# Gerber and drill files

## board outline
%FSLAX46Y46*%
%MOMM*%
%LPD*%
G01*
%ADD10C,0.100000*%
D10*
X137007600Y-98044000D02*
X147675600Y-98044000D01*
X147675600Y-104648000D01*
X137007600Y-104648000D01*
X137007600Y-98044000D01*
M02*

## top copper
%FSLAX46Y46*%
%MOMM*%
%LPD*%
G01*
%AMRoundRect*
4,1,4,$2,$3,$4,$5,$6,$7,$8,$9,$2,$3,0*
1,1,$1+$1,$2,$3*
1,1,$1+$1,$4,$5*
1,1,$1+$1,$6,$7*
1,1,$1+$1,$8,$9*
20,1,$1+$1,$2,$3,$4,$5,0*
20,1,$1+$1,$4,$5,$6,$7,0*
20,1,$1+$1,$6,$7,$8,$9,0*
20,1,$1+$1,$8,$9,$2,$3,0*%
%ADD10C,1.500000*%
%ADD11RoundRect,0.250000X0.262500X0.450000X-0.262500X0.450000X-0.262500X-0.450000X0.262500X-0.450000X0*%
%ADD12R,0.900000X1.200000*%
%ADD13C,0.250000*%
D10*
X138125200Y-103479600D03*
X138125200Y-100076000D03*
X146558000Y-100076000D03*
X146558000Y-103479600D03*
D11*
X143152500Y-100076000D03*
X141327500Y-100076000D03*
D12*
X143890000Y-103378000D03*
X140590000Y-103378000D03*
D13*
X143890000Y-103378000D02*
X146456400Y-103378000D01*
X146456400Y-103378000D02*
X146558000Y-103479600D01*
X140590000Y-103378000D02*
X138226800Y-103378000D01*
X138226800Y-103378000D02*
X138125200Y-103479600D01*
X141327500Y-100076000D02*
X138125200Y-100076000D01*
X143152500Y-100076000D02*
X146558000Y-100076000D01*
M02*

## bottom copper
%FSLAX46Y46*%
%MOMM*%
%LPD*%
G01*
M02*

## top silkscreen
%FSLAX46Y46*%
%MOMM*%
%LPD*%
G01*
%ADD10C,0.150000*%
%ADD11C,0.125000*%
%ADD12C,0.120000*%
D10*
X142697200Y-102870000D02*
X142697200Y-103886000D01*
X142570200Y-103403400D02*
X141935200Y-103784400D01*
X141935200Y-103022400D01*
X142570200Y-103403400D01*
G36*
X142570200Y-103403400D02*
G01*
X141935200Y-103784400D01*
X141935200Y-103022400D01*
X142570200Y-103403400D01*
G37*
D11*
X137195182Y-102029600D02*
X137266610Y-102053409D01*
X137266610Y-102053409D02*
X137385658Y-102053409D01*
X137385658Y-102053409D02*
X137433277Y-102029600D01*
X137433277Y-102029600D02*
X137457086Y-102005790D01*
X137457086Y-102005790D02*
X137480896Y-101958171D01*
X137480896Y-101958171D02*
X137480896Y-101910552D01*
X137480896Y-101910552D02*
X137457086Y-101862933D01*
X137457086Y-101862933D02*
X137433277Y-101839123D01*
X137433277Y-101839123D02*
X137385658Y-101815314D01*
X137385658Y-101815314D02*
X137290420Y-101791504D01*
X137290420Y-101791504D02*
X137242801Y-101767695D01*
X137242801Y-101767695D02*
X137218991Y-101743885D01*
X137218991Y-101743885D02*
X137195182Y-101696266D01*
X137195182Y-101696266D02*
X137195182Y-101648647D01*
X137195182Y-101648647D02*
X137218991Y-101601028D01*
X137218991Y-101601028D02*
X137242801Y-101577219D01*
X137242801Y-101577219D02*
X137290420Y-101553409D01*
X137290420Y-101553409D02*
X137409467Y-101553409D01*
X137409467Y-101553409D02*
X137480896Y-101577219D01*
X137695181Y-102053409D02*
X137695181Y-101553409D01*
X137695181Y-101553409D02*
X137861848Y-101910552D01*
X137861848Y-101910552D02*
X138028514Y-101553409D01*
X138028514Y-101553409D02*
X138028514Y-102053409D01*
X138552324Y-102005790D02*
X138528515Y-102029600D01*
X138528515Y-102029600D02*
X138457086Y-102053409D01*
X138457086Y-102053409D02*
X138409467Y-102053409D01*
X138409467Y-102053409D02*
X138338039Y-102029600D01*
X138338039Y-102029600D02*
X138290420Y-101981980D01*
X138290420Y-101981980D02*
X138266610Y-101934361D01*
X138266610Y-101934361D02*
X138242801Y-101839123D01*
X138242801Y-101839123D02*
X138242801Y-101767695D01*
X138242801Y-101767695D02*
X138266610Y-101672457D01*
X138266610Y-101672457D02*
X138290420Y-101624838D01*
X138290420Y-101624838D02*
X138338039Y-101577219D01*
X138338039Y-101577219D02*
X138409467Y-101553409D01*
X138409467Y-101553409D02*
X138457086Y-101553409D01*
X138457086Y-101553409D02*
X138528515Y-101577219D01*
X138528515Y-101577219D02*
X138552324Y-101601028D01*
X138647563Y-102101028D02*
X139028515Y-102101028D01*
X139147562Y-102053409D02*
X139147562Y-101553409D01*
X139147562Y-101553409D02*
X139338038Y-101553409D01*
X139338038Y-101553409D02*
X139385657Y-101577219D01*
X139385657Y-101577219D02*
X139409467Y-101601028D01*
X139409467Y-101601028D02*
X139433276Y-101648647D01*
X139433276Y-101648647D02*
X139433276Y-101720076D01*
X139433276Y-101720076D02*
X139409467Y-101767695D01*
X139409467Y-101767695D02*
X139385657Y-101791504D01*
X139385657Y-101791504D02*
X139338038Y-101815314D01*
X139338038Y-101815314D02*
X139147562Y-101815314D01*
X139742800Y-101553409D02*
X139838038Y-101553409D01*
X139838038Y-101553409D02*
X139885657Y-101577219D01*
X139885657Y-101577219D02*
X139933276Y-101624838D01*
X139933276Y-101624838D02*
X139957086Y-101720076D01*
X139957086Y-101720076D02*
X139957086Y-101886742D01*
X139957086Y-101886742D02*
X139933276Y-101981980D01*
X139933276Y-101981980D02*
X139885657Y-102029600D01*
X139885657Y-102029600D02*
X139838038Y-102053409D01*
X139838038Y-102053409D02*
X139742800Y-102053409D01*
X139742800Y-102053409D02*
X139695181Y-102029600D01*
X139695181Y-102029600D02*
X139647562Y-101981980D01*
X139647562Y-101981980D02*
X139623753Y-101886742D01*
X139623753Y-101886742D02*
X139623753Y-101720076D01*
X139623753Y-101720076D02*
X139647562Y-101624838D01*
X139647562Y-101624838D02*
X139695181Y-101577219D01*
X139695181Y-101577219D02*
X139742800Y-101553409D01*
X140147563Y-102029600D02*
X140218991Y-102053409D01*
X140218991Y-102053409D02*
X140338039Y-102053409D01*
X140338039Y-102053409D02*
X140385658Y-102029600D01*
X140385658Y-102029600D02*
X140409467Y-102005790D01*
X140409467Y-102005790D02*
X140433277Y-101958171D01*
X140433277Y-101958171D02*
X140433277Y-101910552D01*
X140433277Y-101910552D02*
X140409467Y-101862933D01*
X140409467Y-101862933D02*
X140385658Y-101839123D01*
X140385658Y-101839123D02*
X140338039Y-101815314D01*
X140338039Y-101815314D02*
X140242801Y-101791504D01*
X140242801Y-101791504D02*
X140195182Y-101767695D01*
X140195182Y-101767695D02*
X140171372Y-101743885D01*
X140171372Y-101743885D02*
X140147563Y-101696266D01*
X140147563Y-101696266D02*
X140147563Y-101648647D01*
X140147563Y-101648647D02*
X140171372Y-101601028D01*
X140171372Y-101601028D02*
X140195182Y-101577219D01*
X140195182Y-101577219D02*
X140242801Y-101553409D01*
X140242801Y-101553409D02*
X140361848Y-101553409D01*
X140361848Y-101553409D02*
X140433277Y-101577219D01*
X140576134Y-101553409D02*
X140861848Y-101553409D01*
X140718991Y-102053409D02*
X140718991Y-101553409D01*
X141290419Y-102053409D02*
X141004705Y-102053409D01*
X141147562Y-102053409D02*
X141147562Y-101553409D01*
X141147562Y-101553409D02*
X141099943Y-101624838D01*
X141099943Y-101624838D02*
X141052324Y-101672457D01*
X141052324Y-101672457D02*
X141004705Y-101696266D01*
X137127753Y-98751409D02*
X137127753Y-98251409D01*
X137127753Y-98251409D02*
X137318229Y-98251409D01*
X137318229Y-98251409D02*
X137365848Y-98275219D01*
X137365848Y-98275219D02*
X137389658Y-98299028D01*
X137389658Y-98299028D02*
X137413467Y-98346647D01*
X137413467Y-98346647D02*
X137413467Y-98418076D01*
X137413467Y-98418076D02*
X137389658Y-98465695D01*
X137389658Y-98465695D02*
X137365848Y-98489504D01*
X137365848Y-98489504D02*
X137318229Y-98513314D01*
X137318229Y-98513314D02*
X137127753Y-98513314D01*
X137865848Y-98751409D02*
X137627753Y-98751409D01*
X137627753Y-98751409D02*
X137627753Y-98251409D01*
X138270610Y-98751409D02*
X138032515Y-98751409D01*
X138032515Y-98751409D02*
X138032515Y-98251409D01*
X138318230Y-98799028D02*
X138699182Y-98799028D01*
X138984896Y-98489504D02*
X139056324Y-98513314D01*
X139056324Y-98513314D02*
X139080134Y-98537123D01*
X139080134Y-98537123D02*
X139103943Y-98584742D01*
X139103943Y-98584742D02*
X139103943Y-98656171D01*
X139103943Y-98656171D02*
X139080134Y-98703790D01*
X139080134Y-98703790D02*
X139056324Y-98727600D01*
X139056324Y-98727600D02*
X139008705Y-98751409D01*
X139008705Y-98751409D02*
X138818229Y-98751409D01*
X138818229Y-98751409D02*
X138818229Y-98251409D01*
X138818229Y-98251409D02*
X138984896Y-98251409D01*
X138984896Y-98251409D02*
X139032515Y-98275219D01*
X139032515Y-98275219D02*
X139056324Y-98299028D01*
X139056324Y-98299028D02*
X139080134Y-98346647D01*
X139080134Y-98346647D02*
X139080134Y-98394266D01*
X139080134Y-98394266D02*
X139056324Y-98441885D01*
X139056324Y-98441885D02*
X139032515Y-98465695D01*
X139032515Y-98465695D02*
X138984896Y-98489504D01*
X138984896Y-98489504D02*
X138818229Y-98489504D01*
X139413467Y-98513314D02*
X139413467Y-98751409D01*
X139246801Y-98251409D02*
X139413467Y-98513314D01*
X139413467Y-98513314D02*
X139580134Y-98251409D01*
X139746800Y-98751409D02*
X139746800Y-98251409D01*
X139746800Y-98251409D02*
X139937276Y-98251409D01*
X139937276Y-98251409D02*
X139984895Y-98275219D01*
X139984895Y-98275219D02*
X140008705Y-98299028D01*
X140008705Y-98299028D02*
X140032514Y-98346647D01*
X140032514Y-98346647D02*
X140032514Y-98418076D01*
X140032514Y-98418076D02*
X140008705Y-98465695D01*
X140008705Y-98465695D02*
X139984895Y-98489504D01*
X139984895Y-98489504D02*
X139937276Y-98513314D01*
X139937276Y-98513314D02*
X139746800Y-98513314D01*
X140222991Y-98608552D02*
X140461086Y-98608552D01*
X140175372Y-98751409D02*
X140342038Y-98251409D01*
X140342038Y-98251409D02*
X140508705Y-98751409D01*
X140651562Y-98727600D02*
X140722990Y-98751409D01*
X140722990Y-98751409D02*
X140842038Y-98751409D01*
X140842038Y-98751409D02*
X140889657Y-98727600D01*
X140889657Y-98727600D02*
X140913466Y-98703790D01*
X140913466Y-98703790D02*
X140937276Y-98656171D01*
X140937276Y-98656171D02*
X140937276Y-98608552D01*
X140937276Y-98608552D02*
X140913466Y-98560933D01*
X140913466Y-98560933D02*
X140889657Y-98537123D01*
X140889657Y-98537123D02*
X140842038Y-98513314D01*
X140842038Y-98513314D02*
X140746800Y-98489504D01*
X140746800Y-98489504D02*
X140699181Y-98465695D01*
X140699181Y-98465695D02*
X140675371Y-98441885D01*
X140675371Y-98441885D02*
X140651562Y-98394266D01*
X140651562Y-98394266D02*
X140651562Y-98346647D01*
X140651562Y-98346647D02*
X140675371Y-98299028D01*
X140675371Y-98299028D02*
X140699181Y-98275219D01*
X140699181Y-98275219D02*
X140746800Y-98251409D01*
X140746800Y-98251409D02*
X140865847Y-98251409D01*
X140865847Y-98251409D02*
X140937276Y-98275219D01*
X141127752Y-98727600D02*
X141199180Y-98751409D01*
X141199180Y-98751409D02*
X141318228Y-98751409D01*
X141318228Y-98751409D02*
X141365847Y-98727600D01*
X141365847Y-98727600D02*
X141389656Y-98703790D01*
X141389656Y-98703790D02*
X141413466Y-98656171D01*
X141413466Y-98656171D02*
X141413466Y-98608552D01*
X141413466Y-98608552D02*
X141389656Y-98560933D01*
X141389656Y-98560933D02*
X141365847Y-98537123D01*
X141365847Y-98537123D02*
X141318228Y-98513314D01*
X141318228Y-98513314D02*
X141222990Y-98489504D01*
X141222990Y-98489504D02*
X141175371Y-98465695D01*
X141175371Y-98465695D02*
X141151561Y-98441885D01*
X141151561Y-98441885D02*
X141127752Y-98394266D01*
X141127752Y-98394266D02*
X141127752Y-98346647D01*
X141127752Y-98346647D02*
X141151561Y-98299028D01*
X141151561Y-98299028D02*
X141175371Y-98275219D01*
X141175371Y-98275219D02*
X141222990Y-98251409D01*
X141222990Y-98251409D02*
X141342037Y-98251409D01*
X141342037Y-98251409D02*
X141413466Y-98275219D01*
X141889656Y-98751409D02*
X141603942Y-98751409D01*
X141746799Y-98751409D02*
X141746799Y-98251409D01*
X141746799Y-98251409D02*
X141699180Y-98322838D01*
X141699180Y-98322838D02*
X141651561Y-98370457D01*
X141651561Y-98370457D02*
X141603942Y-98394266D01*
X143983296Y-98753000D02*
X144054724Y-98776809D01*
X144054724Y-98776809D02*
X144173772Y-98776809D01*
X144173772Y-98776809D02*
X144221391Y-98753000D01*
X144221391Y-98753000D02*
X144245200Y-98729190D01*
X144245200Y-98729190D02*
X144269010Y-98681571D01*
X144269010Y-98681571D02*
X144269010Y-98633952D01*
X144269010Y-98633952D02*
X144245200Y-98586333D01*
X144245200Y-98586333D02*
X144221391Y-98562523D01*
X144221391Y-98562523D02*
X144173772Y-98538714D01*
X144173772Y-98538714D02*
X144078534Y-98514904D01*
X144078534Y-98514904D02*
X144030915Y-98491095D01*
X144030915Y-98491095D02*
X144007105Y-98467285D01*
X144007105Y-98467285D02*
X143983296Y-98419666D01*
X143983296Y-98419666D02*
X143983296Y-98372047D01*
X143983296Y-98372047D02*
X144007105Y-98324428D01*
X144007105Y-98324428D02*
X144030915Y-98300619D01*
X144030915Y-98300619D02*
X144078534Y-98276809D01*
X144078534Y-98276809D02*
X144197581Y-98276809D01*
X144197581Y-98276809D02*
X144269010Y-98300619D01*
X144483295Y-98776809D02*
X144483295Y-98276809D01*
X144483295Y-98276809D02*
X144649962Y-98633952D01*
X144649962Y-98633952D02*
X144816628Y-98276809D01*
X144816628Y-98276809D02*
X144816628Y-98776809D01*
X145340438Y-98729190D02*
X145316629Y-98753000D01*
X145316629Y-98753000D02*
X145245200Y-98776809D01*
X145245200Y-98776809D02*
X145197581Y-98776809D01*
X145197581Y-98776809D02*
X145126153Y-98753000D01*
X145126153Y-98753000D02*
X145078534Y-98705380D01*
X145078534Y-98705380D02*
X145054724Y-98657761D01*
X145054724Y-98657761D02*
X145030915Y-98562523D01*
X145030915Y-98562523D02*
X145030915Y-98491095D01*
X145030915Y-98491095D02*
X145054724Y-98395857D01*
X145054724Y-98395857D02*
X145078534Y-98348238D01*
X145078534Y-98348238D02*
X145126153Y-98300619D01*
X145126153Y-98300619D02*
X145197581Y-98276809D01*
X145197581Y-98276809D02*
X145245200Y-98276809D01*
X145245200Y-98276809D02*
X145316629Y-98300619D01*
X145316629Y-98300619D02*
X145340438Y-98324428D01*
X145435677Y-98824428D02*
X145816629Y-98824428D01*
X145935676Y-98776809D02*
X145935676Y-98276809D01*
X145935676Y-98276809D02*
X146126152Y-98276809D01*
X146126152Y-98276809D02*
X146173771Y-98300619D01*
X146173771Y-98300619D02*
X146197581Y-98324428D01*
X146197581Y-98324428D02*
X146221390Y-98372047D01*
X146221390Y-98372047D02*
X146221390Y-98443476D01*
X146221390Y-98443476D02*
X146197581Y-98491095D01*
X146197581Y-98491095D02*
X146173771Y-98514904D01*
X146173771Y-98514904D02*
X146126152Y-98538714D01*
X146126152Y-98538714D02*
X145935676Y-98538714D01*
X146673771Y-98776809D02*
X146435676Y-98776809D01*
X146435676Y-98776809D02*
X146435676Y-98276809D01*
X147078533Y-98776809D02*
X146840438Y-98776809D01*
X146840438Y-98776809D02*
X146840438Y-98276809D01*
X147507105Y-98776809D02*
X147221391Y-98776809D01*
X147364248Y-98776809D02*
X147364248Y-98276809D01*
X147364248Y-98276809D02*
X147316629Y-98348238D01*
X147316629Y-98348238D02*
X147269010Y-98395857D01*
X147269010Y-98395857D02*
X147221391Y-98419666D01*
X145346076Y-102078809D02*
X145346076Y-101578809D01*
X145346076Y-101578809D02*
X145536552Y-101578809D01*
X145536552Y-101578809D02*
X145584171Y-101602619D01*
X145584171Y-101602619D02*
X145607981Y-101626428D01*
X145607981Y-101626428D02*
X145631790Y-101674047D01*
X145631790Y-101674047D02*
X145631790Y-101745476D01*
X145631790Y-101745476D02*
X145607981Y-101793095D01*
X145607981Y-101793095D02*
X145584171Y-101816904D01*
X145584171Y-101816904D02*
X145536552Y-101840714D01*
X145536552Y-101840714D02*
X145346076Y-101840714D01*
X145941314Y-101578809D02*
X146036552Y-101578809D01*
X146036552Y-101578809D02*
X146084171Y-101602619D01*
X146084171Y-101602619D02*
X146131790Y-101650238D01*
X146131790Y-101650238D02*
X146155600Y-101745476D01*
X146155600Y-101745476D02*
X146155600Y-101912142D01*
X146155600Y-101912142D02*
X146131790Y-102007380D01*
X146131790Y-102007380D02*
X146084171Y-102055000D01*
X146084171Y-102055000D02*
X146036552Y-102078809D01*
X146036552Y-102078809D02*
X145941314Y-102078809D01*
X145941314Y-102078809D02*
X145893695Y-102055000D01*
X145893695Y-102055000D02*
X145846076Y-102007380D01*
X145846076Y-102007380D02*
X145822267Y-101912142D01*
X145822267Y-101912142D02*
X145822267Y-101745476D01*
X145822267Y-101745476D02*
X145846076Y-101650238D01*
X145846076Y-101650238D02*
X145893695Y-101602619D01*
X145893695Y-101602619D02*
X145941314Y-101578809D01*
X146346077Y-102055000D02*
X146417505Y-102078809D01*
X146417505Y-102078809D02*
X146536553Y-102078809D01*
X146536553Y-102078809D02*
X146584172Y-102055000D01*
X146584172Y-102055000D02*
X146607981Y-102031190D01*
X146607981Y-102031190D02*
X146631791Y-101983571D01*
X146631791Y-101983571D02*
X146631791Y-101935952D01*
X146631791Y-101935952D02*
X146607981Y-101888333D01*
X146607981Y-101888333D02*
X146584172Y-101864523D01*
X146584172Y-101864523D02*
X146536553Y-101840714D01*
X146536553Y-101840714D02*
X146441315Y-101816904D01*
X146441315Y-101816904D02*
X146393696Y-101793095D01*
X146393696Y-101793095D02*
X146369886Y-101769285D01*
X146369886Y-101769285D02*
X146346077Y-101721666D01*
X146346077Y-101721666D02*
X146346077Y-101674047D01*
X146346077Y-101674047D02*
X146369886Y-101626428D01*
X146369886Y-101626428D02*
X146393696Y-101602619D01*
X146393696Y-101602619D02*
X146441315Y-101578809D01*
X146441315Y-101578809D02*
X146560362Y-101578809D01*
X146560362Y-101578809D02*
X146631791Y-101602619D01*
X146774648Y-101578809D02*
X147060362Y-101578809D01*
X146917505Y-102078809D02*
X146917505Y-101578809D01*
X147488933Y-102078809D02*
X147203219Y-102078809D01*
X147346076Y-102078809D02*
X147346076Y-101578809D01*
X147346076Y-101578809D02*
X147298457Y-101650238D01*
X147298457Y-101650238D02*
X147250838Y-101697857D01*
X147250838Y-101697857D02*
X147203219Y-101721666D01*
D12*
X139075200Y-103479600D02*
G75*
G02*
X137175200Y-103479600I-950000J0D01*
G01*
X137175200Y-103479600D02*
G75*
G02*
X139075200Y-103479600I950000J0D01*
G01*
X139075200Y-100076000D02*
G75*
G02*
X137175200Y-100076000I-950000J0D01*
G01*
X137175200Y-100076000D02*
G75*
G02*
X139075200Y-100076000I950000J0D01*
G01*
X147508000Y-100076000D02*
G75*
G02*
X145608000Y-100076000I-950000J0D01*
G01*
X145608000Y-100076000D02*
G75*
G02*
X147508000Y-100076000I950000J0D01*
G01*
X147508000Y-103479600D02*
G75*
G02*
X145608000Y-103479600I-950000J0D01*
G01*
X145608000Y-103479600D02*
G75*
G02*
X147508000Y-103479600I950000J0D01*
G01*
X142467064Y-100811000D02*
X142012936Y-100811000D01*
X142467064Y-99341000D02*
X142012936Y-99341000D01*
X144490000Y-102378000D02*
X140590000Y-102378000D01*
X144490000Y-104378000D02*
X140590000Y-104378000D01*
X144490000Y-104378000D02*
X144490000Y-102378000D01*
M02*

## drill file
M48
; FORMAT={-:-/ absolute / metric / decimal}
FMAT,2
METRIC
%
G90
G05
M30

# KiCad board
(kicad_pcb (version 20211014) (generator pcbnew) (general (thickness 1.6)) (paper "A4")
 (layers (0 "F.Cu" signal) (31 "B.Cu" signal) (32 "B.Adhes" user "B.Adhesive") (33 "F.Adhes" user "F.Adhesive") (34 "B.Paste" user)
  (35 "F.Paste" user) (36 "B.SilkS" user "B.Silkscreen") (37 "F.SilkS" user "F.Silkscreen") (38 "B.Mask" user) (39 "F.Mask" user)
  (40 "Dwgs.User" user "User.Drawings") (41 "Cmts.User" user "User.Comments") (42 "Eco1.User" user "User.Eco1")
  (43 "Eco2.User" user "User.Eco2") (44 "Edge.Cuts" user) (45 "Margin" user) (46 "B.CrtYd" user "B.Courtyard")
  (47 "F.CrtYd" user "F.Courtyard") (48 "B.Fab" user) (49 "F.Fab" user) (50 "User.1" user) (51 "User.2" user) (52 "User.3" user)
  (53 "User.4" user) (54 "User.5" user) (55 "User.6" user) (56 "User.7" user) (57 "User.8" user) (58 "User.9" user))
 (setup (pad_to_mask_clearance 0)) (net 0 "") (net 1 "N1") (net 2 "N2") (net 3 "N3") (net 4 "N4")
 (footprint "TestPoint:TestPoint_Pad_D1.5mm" (layer "F.Cu") (at 138.1252 103.4796)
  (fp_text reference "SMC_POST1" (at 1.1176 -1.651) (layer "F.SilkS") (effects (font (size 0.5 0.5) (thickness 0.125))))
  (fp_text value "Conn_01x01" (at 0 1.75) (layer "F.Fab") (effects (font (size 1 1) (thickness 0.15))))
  (fp_circle (center 0 0) (end 0 0.95) (layer "F.SilkS") (width 0.12) (fill none))
  (pad "1" smd circle (at 0 0) (size 1.5 1.5) (layers "F.Cu" "F.Mask") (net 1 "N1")))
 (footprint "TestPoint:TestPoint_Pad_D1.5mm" (layer "F.Cu") (at 138.1252 100.076)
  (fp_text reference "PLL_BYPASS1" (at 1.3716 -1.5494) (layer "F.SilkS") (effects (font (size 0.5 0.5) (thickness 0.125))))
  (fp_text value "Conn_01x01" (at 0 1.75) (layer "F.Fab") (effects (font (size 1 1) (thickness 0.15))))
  (fp_circle (center 0 0) (end 0 0.95) (layer "F.SilkS") (width 0.12) (fill none))
  (pad "1" smd circle (at 0 0) (size 1.5 1.5) (layers "F.Cu" "F.Mask") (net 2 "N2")))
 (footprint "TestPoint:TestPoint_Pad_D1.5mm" (layer "F.Cu") (at 146.558 100.076)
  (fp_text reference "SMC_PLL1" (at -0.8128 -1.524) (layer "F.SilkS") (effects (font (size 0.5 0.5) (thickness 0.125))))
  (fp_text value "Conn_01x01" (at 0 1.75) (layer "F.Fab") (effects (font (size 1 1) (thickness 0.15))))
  (fp_circle (center 0 0) (end 0 0.95) (layer "F.SilkS") (width 0.12) (fill none))
  (pad "1" smd circle (at 0 0) (size 1.5 1.5) (layers "F.Cu" "F.Mask") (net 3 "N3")))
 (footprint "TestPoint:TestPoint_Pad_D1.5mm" (layer "F.Cu") (at 146.558 103.4796)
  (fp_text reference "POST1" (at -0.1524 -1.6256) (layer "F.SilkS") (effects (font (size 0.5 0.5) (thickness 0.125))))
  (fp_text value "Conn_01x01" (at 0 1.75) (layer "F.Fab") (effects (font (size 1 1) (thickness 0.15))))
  (fp_circle (center 0 0) (end 0 0.95) (layer "F.SilkS") (width 0.12) (fill none))
  (pad "1" smd circle (at 0 0) (size 1.5 1.5) (layers "F.Cu" "F.Mask") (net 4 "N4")))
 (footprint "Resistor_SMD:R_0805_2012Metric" (layer "F.Cu") (at 142.24 100.076 180)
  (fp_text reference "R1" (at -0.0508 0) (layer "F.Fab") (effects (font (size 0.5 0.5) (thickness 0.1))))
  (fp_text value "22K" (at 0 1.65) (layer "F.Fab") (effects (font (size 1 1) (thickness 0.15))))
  (fp_line (start -0.227064 -0.735) (end 0.227064 -0.735) (layer "F.SilkS") (width 0.12))
  (fp_line (start -0.227064 0.735) (end 0.227064 0.735) (layer "F.SilkS") (width 0.12))
  (pad "1" smd roundrect (at -0.9125 0 180) (size 1.025 1.4) (layers "F.Cu" "F.Paste" "F.Mask") (roundrect_rratio 0.243902439) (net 3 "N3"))
  (pad "2" smd roundrect (at 0.9125 0 180) (size 1.025 1.4) (layers "F.Cu" "F.Paste" "F.Mask") (roundrect_rratio 0.243902439) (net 2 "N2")))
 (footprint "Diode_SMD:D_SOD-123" (layer "F.Cu") (at 142.24 103.378 180)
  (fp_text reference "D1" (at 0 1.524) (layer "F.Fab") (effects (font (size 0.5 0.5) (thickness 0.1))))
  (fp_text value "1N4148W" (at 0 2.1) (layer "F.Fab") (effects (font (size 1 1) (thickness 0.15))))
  (fp_line (start -2.25 1) (end 1.65 1) (layer "F.SilkS") (width 0.12))
  (fp_line (start -2.25 -1) (end 1.65 -1) (layer "F.SilkS") (width 0.12))
  (fp_line (start -2.25 -1) (end -2.25 1) (layer "F.SilkS") (width 0.12))
  (pad "1" smd rect (at -1.65 0 180) (size 0.9 1.2) (layers "F.Cu" "F.Paste" "F.Mask") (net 4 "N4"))
  (pad "2" smd rect (at 1.65 0 180) (size 0.9 1.2) (layers "F.Cu" "F.Paste" "F.Mask") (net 1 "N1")))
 (gr_line (start 142.6972 102.87) (end 142.6972 103.886) (layer "F.SilkS") (width 0.15))
 (gr_poly (pts (xy 142.5702 103.4034) (xy 141.9352 103.7844) (xy 141.9352 103.0224)) (layer "F.SilkS") (width 0.15) (fill solid))
 (gr_rect (start 150.495 106.045) (end 150.495 106.045) (layer "Edge.Cuts") (width 0.1) (fill none))
 (gr_rect (start 137.0076 98.044) (end 147.6756 104.648) (layer "Edge.Cuts") (width 0.1) (fill none))
 (gr_rect (start 147.6756 104.648) (end 147.6756 104.648) (layer "Edge.Cuts") (width 0.1) (fill none))
 (gr_rect (start 150.241 105.791) (end 150.241 105.791) (layer "Edge.Cuts") (width 0.1) (fill none))
 (segment (start 143.89 103.378) (end 146.4564 103.378) (width 0.25) (layer "F.Cu") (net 4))
 (segment (start 146.4564 103.378) (end 146.558 103.4796) (width 0.25) (layer "F.Cu") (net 4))
 (segment (start 140.59 103.378) (end 138.2268 103.378) (width 0.25) (layer "F.Cu") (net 1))
 (segment (start 138.2268 103.378) (end 138.1252 103.4796) (width 0.25) (layer "F.Cu") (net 1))
 (segment (start 141.3275 100.076) (end 138.1252 100.076) (width 0.25) (layer "F.Cu") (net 2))
 (segment (start 143.1525 100.076) (end 146.558 100.076) (width 0.25) (layer "F.Cu") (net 3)))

